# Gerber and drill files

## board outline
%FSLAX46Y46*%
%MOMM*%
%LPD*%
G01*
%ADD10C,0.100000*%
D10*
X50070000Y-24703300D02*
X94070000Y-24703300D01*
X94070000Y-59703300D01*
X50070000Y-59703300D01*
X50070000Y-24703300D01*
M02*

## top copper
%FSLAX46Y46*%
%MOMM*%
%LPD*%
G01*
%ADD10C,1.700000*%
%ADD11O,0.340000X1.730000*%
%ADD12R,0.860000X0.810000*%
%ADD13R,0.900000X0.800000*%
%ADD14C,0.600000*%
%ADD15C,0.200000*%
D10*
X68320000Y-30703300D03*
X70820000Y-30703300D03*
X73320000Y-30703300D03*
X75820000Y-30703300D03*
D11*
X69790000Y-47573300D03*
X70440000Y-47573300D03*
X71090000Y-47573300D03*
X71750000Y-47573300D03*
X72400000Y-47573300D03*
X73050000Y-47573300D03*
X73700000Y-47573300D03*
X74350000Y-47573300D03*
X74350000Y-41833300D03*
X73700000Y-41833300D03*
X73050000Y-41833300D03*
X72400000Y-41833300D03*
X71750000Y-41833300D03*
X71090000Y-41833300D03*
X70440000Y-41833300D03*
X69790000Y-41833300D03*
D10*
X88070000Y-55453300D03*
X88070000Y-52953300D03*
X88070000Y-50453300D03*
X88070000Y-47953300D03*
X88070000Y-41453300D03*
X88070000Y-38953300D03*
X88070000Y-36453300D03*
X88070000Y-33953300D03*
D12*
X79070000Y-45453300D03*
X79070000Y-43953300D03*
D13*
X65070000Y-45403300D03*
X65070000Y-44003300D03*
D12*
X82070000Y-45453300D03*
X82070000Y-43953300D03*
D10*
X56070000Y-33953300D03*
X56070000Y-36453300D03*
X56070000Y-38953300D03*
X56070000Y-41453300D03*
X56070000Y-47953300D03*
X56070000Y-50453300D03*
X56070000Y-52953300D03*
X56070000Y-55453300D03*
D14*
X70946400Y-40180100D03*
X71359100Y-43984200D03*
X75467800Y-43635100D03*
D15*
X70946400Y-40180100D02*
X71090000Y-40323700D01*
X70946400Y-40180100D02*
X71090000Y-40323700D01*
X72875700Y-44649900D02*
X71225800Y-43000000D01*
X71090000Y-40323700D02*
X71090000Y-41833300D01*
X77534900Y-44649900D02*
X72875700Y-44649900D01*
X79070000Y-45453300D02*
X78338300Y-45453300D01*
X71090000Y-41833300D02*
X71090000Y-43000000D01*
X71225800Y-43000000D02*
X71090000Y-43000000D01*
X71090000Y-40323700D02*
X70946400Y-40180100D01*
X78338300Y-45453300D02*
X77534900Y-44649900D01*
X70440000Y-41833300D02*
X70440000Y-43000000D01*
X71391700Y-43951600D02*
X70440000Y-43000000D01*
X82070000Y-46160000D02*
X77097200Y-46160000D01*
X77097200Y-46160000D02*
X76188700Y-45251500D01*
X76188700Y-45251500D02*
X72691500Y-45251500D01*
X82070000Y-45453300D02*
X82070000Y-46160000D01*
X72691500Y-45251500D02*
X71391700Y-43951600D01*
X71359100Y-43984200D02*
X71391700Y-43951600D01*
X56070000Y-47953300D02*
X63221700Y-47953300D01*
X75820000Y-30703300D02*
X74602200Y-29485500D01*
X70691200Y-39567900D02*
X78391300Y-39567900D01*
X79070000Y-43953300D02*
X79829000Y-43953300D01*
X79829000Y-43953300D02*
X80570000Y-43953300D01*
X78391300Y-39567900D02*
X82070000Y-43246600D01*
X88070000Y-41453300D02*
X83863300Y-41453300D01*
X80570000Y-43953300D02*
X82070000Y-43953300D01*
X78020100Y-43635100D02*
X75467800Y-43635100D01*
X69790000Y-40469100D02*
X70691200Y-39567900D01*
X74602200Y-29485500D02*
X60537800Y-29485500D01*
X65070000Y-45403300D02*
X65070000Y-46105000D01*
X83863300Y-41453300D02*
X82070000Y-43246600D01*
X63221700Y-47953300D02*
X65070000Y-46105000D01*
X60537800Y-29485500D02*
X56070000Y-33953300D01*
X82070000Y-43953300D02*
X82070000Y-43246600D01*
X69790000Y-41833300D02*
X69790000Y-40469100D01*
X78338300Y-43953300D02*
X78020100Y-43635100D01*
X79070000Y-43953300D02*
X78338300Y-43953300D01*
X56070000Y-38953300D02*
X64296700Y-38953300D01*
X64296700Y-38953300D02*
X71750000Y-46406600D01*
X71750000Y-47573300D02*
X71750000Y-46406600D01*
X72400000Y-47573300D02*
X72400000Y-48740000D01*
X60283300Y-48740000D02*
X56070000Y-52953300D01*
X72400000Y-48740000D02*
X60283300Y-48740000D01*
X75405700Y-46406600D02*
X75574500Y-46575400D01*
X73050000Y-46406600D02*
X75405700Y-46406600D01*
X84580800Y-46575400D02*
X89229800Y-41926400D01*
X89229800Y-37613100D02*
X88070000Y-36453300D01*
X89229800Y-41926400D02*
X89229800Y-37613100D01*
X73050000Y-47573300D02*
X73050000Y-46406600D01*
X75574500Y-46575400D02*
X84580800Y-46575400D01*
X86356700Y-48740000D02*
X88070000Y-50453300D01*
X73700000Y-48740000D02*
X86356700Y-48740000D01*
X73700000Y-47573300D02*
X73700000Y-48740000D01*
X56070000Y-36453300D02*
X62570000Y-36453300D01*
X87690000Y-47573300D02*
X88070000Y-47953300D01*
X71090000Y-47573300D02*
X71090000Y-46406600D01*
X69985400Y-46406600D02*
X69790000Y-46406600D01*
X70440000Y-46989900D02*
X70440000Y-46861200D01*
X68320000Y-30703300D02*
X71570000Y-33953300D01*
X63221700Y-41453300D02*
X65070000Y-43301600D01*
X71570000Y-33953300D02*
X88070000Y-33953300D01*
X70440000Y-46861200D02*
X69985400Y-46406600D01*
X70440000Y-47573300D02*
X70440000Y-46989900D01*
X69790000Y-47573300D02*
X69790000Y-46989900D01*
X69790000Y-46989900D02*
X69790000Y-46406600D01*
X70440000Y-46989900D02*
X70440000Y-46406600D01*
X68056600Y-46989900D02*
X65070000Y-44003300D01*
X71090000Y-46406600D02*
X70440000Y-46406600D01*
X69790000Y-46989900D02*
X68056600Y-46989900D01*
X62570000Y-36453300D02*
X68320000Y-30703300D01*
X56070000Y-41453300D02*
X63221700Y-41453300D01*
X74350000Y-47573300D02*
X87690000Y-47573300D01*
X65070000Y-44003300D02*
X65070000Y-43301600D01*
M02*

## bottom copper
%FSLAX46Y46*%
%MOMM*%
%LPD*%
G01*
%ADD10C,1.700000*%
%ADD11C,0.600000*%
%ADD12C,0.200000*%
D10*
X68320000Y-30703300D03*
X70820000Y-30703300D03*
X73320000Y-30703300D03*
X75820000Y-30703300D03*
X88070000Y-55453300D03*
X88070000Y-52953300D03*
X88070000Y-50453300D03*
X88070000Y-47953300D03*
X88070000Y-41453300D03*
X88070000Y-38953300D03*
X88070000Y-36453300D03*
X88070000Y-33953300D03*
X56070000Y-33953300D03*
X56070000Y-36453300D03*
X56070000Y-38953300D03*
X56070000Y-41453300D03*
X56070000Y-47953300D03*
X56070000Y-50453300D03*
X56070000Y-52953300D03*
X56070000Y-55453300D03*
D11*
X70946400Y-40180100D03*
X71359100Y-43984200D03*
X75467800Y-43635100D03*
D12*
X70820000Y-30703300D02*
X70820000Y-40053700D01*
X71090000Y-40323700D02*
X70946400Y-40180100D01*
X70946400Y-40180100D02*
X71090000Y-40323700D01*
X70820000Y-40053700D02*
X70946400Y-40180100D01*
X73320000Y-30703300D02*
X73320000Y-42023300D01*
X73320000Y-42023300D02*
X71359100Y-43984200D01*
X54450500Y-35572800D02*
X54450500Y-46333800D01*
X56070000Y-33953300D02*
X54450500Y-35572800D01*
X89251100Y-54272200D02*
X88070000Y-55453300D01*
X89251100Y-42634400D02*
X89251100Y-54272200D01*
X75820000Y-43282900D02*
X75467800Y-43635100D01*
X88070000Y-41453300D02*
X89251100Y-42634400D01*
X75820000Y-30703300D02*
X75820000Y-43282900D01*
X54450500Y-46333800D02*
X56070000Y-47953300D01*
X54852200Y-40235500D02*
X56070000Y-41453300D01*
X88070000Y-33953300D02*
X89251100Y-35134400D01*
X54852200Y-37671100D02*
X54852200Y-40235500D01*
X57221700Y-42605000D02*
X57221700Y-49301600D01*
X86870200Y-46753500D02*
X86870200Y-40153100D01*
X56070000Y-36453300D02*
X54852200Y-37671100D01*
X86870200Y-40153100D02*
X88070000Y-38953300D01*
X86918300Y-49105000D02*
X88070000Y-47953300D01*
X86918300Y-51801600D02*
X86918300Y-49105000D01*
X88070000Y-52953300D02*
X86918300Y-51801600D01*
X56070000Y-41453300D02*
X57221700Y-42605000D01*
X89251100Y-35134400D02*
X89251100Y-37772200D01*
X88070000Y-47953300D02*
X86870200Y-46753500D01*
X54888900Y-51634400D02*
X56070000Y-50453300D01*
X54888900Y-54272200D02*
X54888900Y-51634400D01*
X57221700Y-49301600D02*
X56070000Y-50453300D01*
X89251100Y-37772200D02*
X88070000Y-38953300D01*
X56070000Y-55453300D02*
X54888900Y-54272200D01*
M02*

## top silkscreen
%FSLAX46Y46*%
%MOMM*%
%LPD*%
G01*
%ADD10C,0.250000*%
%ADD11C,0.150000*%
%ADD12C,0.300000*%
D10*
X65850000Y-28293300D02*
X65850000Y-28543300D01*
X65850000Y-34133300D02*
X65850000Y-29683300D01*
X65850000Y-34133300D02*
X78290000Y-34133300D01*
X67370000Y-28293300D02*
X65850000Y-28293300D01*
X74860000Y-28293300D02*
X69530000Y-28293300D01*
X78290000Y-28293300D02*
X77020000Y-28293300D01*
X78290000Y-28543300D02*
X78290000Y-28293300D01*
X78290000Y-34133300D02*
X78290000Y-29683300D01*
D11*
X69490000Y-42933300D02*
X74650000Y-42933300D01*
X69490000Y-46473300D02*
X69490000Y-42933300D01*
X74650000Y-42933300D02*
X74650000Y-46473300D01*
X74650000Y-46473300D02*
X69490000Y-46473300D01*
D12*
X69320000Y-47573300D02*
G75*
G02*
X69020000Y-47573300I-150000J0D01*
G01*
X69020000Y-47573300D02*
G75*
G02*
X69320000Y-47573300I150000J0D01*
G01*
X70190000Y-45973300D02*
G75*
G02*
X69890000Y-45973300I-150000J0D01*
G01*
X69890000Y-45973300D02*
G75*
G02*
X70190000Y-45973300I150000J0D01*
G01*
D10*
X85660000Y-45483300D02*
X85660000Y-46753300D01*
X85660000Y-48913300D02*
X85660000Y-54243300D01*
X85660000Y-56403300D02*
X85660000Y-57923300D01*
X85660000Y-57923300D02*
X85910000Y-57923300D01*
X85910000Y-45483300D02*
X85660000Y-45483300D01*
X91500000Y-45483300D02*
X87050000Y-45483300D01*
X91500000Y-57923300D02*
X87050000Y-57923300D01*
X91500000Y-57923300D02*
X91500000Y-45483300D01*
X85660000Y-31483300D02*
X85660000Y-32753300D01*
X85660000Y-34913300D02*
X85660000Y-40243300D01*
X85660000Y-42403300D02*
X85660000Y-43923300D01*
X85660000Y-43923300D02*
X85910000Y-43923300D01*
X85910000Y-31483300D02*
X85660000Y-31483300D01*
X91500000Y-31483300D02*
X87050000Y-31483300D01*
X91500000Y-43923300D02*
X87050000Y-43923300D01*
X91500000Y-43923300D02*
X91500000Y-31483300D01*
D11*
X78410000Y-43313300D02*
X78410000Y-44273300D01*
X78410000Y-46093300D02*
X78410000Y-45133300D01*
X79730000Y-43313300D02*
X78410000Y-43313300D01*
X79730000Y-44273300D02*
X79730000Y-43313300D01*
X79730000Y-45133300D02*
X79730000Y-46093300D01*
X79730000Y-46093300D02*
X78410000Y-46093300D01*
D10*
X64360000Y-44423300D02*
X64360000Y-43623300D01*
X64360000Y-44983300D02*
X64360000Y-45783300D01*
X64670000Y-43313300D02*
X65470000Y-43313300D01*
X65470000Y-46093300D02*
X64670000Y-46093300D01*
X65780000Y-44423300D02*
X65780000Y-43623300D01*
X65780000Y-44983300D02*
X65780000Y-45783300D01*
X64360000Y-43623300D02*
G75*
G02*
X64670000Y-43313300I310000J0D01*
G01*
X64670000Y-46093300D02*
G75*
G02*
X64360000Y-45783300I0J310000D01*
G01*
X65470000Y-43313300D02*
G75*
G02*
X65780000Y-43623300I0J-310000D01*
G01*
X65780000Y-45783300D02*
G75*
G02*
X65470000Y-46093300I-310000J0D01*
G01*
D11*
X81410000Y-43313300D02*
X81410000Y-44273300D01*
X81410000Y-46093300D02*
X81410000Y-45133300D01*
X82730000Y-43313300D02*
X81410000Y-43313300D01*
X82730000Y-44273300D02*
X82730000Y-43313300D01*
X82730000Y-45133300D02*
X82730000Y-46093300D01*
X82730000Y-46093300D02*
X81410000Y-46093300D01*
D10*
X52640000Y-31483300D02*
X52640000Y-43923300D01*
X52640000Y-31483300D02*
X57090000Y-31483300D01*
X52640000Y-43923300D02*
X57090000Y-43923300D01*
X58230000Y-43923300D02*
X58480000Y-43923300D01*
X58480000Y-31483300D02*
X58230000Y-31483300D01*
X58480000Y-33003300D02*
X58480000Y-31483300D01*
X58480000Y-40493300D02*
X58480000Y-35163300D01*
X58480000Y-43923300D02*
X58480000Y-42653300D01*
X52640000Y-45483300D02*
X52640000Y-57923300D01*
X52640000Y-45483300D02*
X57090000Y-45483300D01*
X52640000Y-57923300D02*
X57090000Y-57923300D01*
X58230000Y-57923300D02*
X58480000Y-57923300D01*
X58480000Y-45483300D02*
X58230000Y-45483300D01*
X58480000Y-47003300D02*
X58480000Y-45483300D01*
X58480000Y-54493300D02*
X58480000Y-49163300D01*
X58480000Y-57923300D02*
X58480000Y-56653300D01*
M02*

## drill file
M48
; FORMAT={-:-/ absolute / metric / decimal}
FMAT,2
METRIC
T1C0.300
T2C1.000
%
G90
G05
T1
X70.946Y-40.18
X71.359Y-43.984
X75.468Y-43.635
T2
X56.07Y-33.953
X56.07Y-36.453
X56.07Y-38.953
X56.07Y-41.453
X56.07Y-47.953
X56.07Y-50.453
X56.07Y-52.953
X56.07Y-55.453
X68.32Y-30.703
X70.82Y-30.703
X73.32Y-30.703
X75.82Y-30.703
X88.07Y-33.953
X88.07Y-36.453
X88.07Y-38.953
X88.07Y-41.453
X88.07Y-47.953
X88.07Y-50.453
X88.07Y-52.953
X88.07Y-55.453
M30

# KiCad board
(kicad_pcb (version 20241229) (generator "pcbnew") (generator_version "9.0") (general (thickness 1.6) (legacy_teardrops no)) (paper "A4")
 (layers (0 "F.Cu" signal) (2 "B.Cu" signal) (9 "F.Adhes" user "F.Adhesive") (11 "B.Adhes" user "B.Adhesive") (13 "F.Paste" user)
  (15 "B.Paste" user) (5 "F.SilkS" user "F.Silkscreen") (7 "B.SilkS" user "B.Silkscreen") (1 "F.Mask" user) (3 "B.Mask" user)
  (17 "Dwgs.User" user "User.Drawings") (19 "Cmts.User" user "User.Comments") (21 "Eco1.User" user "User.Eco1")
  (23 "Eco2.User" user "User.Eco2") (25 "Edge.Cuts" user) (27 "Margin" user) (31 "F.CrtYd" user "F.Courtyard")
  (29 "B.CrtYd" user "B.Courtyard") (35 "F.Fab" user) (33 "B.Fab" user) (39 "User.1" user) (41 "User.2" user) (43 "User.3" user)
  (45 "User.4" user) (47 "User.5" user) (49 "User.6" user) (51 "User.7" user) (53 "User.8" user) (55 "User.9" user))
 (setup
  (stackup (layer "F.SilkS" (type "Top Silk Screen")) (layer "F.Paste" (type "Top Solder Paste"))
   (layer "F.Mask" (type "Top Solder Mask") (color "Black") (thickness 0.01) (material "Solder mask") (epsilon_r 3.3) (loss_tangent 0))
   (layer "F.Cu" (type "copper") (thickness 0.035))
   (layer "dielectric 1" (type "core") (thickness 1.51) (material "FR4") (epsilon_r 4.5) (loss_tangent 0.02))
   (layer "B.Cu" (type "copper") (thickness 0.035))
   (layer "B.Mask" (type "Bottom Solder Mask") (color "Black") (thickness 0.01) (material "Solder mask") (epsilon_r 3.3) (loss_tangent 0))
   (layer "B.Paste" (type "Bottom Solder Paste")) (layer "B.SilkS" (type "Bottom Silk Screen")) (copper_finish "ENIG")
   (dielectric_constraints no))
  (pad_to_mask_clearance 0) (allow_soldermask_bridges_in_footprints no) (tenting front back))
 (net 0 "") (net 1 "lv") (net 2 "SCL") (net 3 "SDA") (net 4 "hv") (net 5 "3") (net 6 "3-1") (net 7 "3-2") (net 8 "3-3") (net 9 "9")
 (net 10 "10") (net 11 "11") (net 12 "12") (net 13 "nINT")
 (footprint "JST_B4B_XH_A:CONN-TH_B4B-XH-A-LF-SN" (layer "F.Cu") (at 72.07 30.7033 180)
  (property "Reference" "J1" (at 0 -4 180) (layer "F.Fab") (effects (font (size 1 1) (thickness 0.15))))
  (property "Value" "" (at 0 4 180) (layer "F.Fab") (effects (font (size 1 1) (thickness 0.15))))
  (fp_line (start 6.22 2.41) (end 6.22 2.16) (stroke (width 0.25) (type solid)) (layer "F.SilkS"))
  (fp_line (start 6.22 -3.43) (end 6.22 1.02) (stroke (width 0.25) (type solid)) (layer "F.SilkS"))
  (fp_line (start 6.22 -3.43) (end -6.22 -3.43) (stroke (width 0.25) (type solid)) (layer "F.SilkS"))
  (fp_line (start 4.7 2.41) (end 6.22 2.41) (stroke (width 0.25) (type solid)) (layer "F.SilkS"))
  (fp_line (start -2.79 2.41) (end 2.54 2.41) (stroke (width 0.25) (type solid)) (layer "F.SilkS"))
  (fp_line (start -6.22 2.41) (end -4.95 2.41) (stroke (width 0.25) (type solid)) (layer "F.SilkS"))
  (fp_line (start -6.22 2.16) (end -6.22 2.41) (stroke (width 0.25) (type solid)) (layer "F.SilkS"))
  (fp_line (start -6.22 -3.43) (end -6.22 1.02) (stroke (width 0.25) (type solid)) (layer "F.SilkS"))
  (pad "1" thru_hole circle (at 3.75 0 180) (size 1.7 1.7) (drill 0.999998) (layers "*.Cu" "*.Mask") (remove_unused_layers no) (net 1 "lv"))
  (pad "2" thru_hole circle (at 1.25 0 180) (size 1.7 1.7) (drill 0.999998) (layers "*.Cu" "*.Mask") (remove_unused_layers no) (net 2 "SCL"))
  (pad "3" thru_hole circle (at -1.25 0 180) (size 1.7 1.7) (drill 0.999998) (layers "*.Cu" "*.Mask") (remove_unused_layers no)
   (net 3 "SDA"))
  (pad "4" thru_hole circle (at -3.75 0 180) (size 1.7 1.7) (drill 0.999998) (layers "*.Cu" "*.Mask") (remove_unused_layers no) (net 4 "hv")))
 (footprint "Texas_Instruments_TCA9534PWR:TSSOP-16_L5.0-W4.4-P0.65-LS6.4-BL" (layer "F.Cu") (at 72.07 44.7033)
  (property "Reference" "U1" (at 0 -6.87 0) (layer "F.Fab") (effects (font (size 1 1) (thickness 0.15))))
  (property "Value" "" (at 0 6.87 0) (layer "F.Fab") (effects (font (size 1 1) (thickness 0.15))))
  (fp_line (start -2.58 -1.77) (end 2.58 -1.77) (stroke (width 0.15) (type solid)) (layer "F.SilkS"))
  (fp_line (start -2.58 1.77) (end -2.58 -1.77) (stroke (width 0.15) (type solid)) (layer "F.SilkS"))
  (fp_line (start 2.58 -1.77) (end 2.58 1.77) (stroke (width 0.15) (type solid)) (layer "F.SilkS"))
  (fp_line (start 2.58 1.77) (end -2.58 1.77) (stroke (width 0.15) (type solid)) (layer "F.SilkS"))
  (fp_circle (center -2.9 2.87) (end -2.75 2.87) (stroke (width 0.3) (type solid)) (fill no) (layer "F.SilkS"))
  (fp_circle (center -2.03 1.27) (end -1.88 1.27) (stroke (width 0.3) (type solid)) (fill no) (layer "F.SilkS"))
  (pad "1" smd oval (at -2.28 2.87) (size 0.34 1.73) (layers "F.Cu" "F.Mask" "F.Paste") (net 1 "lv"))
  (pad "2" smd oval (at -1.63 2.87) (size 0.34 1.73) (layers "F.Cu" "F.Mask" "F.Paste") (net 1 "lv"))
  (pad "3" smd oval (at -0.98 2.87) (size 0.34 1.73) (layers "F.Cu" "F.Mask" "F.Paste") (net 1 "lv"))
  (pad "4" smd oval (at -0.32 2.87) (size 0.34 1.73) (layers "F.Cu" "F.Mask" "F.Paste") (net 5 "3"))
  (pad "5" smd oval (at 0.33 2.87) (size 0.34 1.73) (layers "F.Cu" "F.Mask" "F.Paste") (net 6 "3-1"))
  (pad "6" smd oval (at 0.98 2.87) (size 0.34 1.73) (layers "F.Cu" "F.Mask" "F.Paste") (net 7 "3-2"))
  (pad "7" smd oval (at 1.63 2.87) (size 0.34 1.73) (layers "F.Cu" "F.Mask" "F.Paste") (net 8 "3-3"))
  (pad "8" smd oval (at 2.28 2.87) (size 0.34 1.73) (layers "F.Cu" "F.Mask" "F.Paste") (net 1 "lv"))
  (pad "9" smd oval (at 2.28 -2.87) (size 0.34 1.73) (layers "F.Cu" "F.Mask" "F.Paste") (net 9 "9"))
  (pad "10" smd oval (at 1.63 -2.87) (size 0.34 1.73) (layers "F.Cu" "F.Mask" "F.Paste") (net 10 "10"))
  (pad "11" smd oval (at 0.98 -2.87) (size 0.34 1.73) (layers "F.Cu" "F.Mask" "F.Paste") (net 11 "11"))
  (pad "12" smd oval (at 0.33 -2.87) (size 0.34 1.73) (layers "F.Cu" "F.Mask" "F.Paste") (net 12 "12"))
  (pad "13" smd oval (at -0.32 -2.87) (size 0.34 1.73) (layers "F.Cu" "F.Mask" "F.Paste") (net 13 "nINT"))
  (pad "14" smd oval (at -0.98 -2.87) (size 0.34 1.73) (layers "F.Cu" "F.Mask" "F.Paste") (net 2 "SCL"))
  (pad "15" smd oval (at -1.63 -2.87) (size 0.34 1.73) (layers "F.Cu" "F.Mask" "F.Paste") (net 3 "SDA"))
  (pad "16" smd oval (at -2.28 -2.87) (size 0.34 1.73) (layers "F.Cu" "F.Mask" "F.Paste") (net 4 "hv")))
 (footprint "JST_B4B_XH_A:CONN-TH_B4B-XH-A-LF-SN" (layer "F.Cu") (at 88.07 51.7033 -90)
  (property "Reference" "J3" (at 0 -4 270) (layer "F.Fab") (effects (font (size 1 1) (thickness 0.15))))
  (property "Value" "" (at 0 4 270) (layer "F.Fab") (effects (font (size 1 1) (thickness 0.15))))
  (fp_line (start -6.22 2.41) (end -4.95 2.41) (stroke (width 0.25) (type solid)) (layer "F.SilkS"))
  (fp_line (start -2.79 2.41) (end 2.54 2.41) (stroke (width 0.25) (type solid)) (layer "F.SilkS"))
  (fp_line (start 4.7 2.41) (end 6.22 2.41) (stroke (width 0.25) (type solid)) (layer "F.SilkS"))
  (fp_line (start 6.22 2.41) (end 6.22 2.16) (stroke (width 0.25) (type solid)) (layer "F.SilkS"))
  (fp_line (start -6.22 2.16) (end -6.22 2.41) (stroke (width 0.25) (type solid)) (layer "F.SilkS"))
  (fp_line (start -6.22 -3.43) (end -6.22 1.02) (stroke (width 0.25) (type solid)) (layer "F.SilkS"))
  (fp_line (start 6.22 -3.43) (end 6.22 1.02) (stroke (width 0.25) (type solid)) (layer "F.SilkS"))
  (fp_line (start 6.22 -3.43) (end -6.22 -3.43) (stroke (width 0.25) (type solid)) (layer "F.SilkS"))
  (pad "1" thru_hole circle (at 3.75 0 270) (size 1.7 1.7) (drill 0.999998) (layers "*.Cu" "*.Mask") (remove_unused_layers no) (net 4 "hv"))
  (pad "2" thru_hole circle (at 1.25 0 270) (size 1.7 1.7) (drill 0.999998) (layers "*.Cu" "*.Mask") (remove_unused_layers no) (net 1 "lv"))
  (pad "3" thru_hole circle (at -1.25 0 270) (size 1.7 1.7) (drill 0.999998) (layers "*.Cu" "*.Mask") (remove_unused_layers no)
   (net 8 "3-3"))
  (pad "4" thru_hole circle (at -3.75 0 270) (size 1.7 1.7) (drill 0.999998) (layers "*.Cu" "*.Mask") (remove_unused_layers no) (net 1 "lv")))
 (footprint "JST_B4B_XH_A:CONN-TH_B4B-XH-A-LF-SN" (layer "F.Cu") (at 88.07 37.7033 -90)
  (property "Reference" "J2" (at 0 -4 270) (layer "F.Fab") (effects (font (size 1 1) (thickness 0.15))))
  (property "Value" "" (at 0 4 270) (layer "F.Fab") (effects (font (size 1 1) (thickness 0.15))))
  (fp_line (start -6.22 2.41) (end -4.95 2.41) (stroke (width 0.25) (type solid)) (layer "F.SilkS"))
  (fp_line (start -2.79 2.41) (end 2.54 2.41) (stroke (width 0.25) (type solid)) (layer "F.SilkS"))
  (fp_line (start 4.7 2.41) (end 6.22 2.41) (stroke (width 0.25) (type solid)) (layer "F.SilkS"))
  (fp_line (start 6.22 2.41) (end 6.22 2.16) (stroke (width 0.25) (type solid)) (layer "F.SilkS"))
  (fp_line (start -6.22 2.16) (end -6.22 2.41) (stroke (width 0.25) (type solid)) (layer "F.SilkS"))
  (fp_line (start -6.22 -3.43) (end -6.22 1.02) (stroke (width 0.25) (type solid)) (layer "F.SilkS"))
  (fp_line (start 6.22 -3.43) (end 6.22 1.02) (stroke (width 0.25) (type solid)) (layer "F.SilkS"))
  (fp_line (start 6.22 -3.43) (end -6.22 -3.43) (stroke (width 0.25) (type solid)) (layer "F.SilkS"))
  (pad "1" thru_hole circle (at 3.75 0 270) (size 1.7 1.7) (drill 0.999998) (layers "*.Cu" "*.Mask") (remove_unused_layers no) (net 4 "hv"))
  (pad "2" thru_hole circle (at 1.25 0 270) (size 1.7 1.7) (drill 0.999998) (layers "*.Cu" "*.Mask") (remove_unused_layers no) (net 1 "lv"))
  (pad "3" thru_hole circle (at -1.25 0 270) (size 1.7 1.7) (drill 0.999998) (layers "*.Cu" "*.Mask") (remove_unused_layers no)
   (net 7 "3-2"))
  (pad "4" thru_hole circle (at -3.75 0 270) (size 1.7 1.7) (drill 0.999998) (layers "*.Cu" "*.Mask") (remove_unused_layers no) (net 1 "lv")))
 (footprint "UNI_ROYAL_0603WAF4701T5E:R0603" (layer "F.Cu") (at 79.07 44.7033 90)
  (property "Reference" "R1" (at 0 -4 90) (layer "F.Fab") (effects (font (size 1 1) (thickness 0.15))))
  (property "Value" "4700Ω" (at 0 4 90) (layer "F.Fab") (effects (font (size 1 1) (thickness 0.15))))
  (fp_line (start 1.39 -0.66) (end 0.43 -0.66) (stroke (width 0.15) (type solid)) (layer "F.SilkS"))
  (fp_line (start -1.39 -0.66) (end -0.43 -0.66) (stroke (width 0.15) (type solid)) (layer "F.SilkS"))
  (fp_line (start 1.39 0.66) (end 1.39 -0.66) (stroke (width 0.15) (type solid)) (layer "F.SilkS"))
  (fp_line (start 0.43 0.66) (end 1.39 0.66) (stroke (width 0.15) (type solid)) (layer "F.SilkS"))
  (fp_line (start -0.43 0.66) (end -1.39 0.66) (stroke (width 0.15) (type solid)) (layer "F.SilkS"))
  (fp_line (start -1.39 0.66) (end -1.39 -0.66) (stroke (width 0.15) (type solid)) (layer "F.SilkS"))
  (pad "1" smd rect (at -0.75 0 90) (size 0.81 0.86) (layers "F.Cu" "F.Mask" "F.Paste") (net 2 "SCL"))
  (pad "2" smd rect (at 0.75 0 90) (size 0.81 0.86) (layers "F.Cu" "F.Mask" "F.Paste") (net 4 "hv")))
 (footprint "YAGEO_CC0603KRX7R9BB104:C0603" (layer "F.Cu") (at 65.07 44.7033 90)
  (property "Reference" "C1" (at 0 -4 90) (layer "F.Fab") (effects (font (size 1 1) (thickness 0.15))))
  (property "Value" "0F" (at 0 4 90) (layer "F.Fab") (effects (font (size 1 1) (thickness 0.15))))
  (fp_line (start 0.28 -0.71) (end 1.08 -0.71) (stroke (width 0.25) (type solid)) (layer "F.SilkS"))
  (fp_line (start -0.28 -0.71) (end -1.08 -0.71) (stroke (width 0.25) (type solid)) (layer "F.SilkS"))
  (fp_line (start 1.39 -0.4) (end 1.39 0.4) (stroke (width 0.25) (type solid)) (layer "F.SilkS"))
  (fp_line (start -1.39 0.4) (end -1.39 -0.4) (stroke (width 0.25) (type solid)) (layer "F.SilkS"))
  (fp_line (start 0.28 0.71) (end 1.08 0.71) (stroke (width 0.25) (type solid)) (layer "F.SilkS"))
  (fp_line (start -0.28 0.71) (end -1.08 0.71) (stroke (width 0.25) (type solid)) (layer "F.SilkS"))
  (fp_arc (start 1.08 -0.71) (mid 1.299203 -0.619203) (end 1.39 -0.4) (stroke (width 0.25) (type solid)) (layer "F.SilkS"))
  (fp_arc (start -1.39 -0.4) (mid -1.299203 -0.619203) (end -1.08 -0.71) (stroke (width 0.25) (type solid)) (layer "F.SilkS"))
  (fp_arc (start 1.39 0.4) (mid 1.299203 0.619203) (end 1.08 0.71) (stroke (width 0.25) (type solid)) (layer "F.SilkS"))
  (fp_arc (start -1.08 0.71) (mid -1.299203 0.619203) (end -1.39 0.4) (stroke (width 0.25) (type solid)) (layer "F.SilkS"))
  (pad "1" smd rect (at -0.7 0 90) (size 0.8 0.9) (layers "F.Cu" "F.Mask" "F.Paste") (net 4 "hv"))
  (pad "2" smd rect (at 0.7 0 90) (size 0.8 0.9) (layers "F.Cu" "F.Mask" "F.Paste") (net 1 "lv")))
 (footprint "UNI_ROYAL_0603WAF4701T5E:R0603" (layer "F.Cu") (at 82.07 44.7033 90)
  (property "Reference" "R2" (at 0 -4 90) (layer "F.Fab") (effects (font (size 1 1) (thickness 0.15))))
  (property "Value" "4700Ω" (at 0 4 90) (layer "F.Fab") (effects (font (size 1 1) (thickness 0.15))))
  (fp_line (start 1.39 -0.66) (end 0.43 -0.66) (stroke (width 0.15) (type solid)) (layer "F.SilkS"))
  (fp_line (start -1.39 -0.66) (end -0.43 -0.66) (stroke (width 0.15) (type solid)) (layer "F.SilkS"))
  (fp_line (start 1.39 0.66) (end 1.39 -0.66) (stroke (width 0.15) (type solid)) (layer "F.SilkS"))
  (fp_line (start 0.43 0.66) (end 1.39 0.66) (stroke (width 0.15) (type solid)) (layer "F.SilkS"))
  (fp_line (start -0.43 0.66) (end -1.39 0.66) (stroke (width 0.15) (type solid)) (layer "F.SilkS"))
  (fp_line (start -1.39 0.66) (end -1.39 -0.66) (stroke (width 0.15) (type solid)) (layer "F.SilkS"))
  (pad "1" smd rect (at -0.75 0 90) (size 0.81 0.86) (layers "F.Cu" "F.Mask" "F.Paste") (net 3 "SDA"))
  (pad "2" smd rect (at 0.75 0 90) (size 0.81 0.86) (layers "F.Cu" "F.Mask" "F.Paste") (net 4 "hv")))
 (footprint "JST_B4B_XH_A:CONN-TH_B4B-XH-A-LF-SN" (layer "F.Cu") (at 56.07 37.7033 90)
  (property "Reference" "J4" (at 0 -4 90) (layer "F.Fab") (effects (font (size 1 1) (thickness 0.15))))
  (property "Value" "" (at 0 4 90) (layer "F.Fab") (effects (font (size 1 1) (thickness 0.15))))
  (fp_line (start 6.22 -3.43) (end -6.22 -3.43) (stroke (width 0.25) (type solid)) (layer "F.SilkS"))
  (fp_line (start 6.22 -3.43) (end 6.22 1.02) (stroke (width 0.25) (type solid)) (layer "F.SilkS"))
  (fp_line (start -6.22 -3.43) (end -6.22 1.02) (stroke (width 0.25) (type solid)) (layer "F.SilkS"))
  (fp_line (start -6.22 2.16) (end -6.22 2.41) (stroke (width 0.25) (type solid)) (layer "F.SilkS"))
  (fp_line (start 6.22 2.41) (end 6.22 2.16) (stroke (width 0.25) (type solid)) (layer "F.SilkS"))
  (fp_line (start 4.7 2.41) (end 6.22 2.41) (stroke (width 0.25) (type solid)) (layer "F.SilkS"))
  (fp_line (start -2.79 2.41) (end 2.54 2.41) (stroke (width 0.25) (type solid)) (layer "F.SilkS"))
  (fp_line (start -6.22 2.41) (end -4.95 2.41) (stroke (width 0.25) (type solid)) (layer "F.SilkS"))
  (pad "1" thru_hole circle (at 3.75 0 90) (size 1.7 1.7) (drill 0.999998) (layers "*.Cu" "*.Mask") (remove_unused_layers no) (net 4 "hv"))
  (pad "2" thru_hole circle (at 1.25 0 90) (size 1.7 1.7) (drill 0.999998) (layers "*.Cu" "*.Mask") (remove_unused_layers no) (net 1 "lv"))
  (pad "3" thru_hole circle (at -1.25 0 90) (size 1.7 1.7) (drill 0.999998) (layers "*.Cu" "*.Mask") (remove_unused_layers no) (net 5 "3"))
  (pad "4" thru_hole circle (at -3.75 0 90) (size 1.7 1.7) (drill 0.999998) (layers "*.Cu" "*.Mask") (remove_unused_layers no) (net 1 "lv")))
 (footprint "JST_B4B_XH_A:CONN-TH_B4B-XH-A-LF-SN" (layer "F.Cu") (at 56.07 51.7033 90)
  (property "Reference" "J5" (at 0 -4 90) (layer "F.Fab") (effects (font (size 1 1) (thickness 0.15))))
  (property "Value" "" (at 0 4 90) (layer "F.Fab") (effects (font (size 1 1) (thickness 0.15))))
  (fp_line (start 6.22 -3.43) (end -6.22 -3.43) (stroke (width 0.25) (type solid)) (layer "F.SilkS"))
  (fp_line (start 6.22 -3.43) (end 6.22 1.02) (stroke (width 0.25) (type solid)) (layer "F.SilkS"))
  (fp_line (start -6.22 -3.43) (end -6.22 1.02) (stroke (width 0.25) (type solid)) (layer "F.SilkS"))
  (fp_line (start -6.22 2.16) (end -6.22 2.41) (stroke (width 0.25) (type solid)) (layer "F.SilkS"))
  (fp_line (start 6.22 2.41) (end 6.22 2.16) (stroke (width 0.25) (type solid)) (layer "F.SilkS"))
  (fp_line (start 4.7 2.41) (end 6.22 2.41) (stroke (width 0.25) (type solid)) (layer "F.SilkS"))
  (fp_line (start -2.79 2.41) (end 2.54 2.41) (stroke (width 0.25) (type solid)) (layer "F.SilkS"))
  (fp_line (start -6.22 2.41) (end -4.95 2.41) (stroke (width 0.25) (type solid)) (layer "F.SilkS"))
  (pad "1" thru_hole circle (at 3.75 0 90) (size 1.7 1.7) (drill 0.999998) (layers "*.Cu" "*.Mask") (remove_unused_layers no) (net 4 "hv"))
  (pad "2" thru_hole circle (at 1.25 0 90) (size 1.7 1.7) (drill 0.999998) (layers "*.Cu" "*.Mask") (remove_unused_layers no) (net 1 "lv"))
  (pad "3" thru_hole circle (at -1.25 0 90) (size 1.7 1.7) (drill 0.999998) (layers "*.Cu" "*.Mask") (remove_unused_layers no) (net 6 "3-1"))
  (pad "4" thru_hole circle (at -3.75 0 90) (size 1.7 1.7) (drill 0.999998) (layers "*.Cu" "*.Mask") (remove_unused_layers no) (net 1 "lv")))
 (gr_rect (start 50.07 24.7033) (end 94.07 59.7033) (stroke (width 0.1) (type solid)) (fill no) (layer "Edge.Cuts"))
 (segment (start 70.9464 40.1801) (end 71.09 40.3237) (width 0.2) (layer "F.Cu") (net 2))
 (segment (start 70.9464 40.1801) (end 71.09 40.3237) (width 0.2) (layer "F.Cu") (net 2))
 (segment (start 72.8757 44.6499) (end 71.2258 43) (width 0.2) (layer "F.Cu") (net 2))
 (segment (start 71.09 40.3237) (end 71.09 41.8333) (width 0.2) (layer "F.Cu") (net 2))
 (segment (start 77.5349 44.6499) (end 72.8757 44.6499) (width 0.2) (layer "F.Cu") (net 2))
 (segment (start 79.07 45.4533) (end 78.3383 45.4533) (width 0.2) (layer "F.Cu") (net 2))
 (segment (start 71.09 41.8333) (end 71.09 43) (width 0.2) (layer "F.Cu") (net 2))
 (segment (start 71.2258 43) (end 71.09 43) (width 0.2) (layer "F.Cu") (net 2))
 (segment (start 71.09 40.3237) (end 70.9464 40.1801) (width 0.2) (layer "F.Cu") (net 2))
 (segment (start 78.3383 45.4533) (end 77.5349 44.6499) (width 0.2) (layer "F.Cu") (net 2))
 (via (at 70.9464 40.1801) (size 0.6) (drill 0.3) (layers "F.Cu" "B.Cu") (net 2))
 (segment (start 70.82 30.7033) (end 70.82 40.0537) (width 0.2) (layer "B.Cu") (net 2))
 (segment (start 71.09 40.3237) (end 70.9464 40.1801) (width 0.2) (layer "B.Cu") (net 2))
 (segment (start 70.9464 40.1801) (end 71.09 40.3237) (width 0.2) (layer "B.Cu") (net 2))
 (segment (start 70.82 40.0537) (end 70.9464 40.1801) (width 0.2) (layer "B.Cu") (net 2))
 (segment (start 70.44 41.8333) (end 70.44 43) (width 0.2) (layer "F.Cu") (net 3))
 (segment (start 71.3917 43.9516) (end 70.44 43) (width 0.2) (layer "F.Cu") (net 3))
 (segment (start 82.07 46.16) (end 77.0972 46.16) (width 0.2) (layer "F.Cu") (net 3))
 (segment (start 77.0972 46.16) (end 76.1887 45.2515) (width 0.2) (layer "F.Cu") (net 3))
 (segment (start 76.1887 45.2515) (end 72.6915 45.2515) (width 0.2) (layer "F.Cu") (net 3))
 (segment (start 82.07 45.4533) (end 82.07 46.16) (width 0.2) (layer "F.Cu") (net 3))
 (segment (start 72.6915 45.2515) (end 71.3917 43.9516) (width 0.2) (layer "F.Cu") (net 3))
 (segment (start 71.3591 43.9842) (end 71.3917 43.9516) (width 0.2) (layer "F.Cu") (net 3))
 (via (at 71.3591 43.9842) (size 0.6) (drill 0.3) (layers "F.Cu" "B.Cu") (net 3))
 (segment (start 73.32 30.7033) (end 73.32 42.0233) (width 0.2) (layer "B.Cu") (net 3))
 (segment (start 73.32 42.0233) (end 71.3591 43.9842) (width 0.2) (layer "B.Cu") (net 3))
 (segment (start 56.07 47.9533) (end 63.2217 47.9533) (width 0.2) (layer "F.Cu") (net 4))
 (segment (start 75.82 30.7033) (end 74.6022 29.4855) (width 0.2) (layer "F.Cu") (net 4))
 (segment (start 70.6912 39.5679) (end 78.3913 39.5679) (width 0.2) (layer "F.Cu") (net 4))
 (segment (start 79.07 43.9533) (end 79.829 43.9533) (width 0.2) (layer "F.Cu") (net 4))
 (segment (start 79.829 43.9533) (end 80.57 43.9533) (width 0.2) (layer "F.Cu") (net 4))
 (segment (start 78.3913 39.5679) (end 82.07 43.2466) (width 0.2) (layer "F.Cu") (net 4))
 (segment (start 88.07 41.4533) (end 83.8633 41.4533) (width 0.2) (layer "F.Cu") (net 4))
 (segment (start 80.57 43.9533) (end 82.07 43.9533) (width 0.2) (layer "F.Cu") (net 4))
 (segment (start 78.0201 43.6351) (end 75.4678 43.6351) (width 0.2) (layer "F.Cu") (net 4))
 (segment (start 69.79 40.4691) (end 70.6912 39.5679) (width 0.2) (layer "F.Cu") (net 4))
 (segment (start 74.6022 29.4855) (end 60.5378 29.4855) (width 0.2) (layer "F.Cu") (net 4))
 (segment (start 65.07 45.4033) (end 65.07 46.105) (width 0.2) (layer "F.Cu") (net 4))
 (segment (start 83.8633 41.4533) (end 82.07 43.2466) (width 0.2) (layer "F.Cu") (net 4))
 (segment (start 63.2217 47.9533) (end 65.07 46.105) (width 0.2) (layer "F.Cu") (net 4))
 (segment (start 60.5378 29.4855) (end 56.07 33.9533) (width 0.2) (layer "F.Cu") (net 4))
 (segment (start 82.07 43.9533) (end 82.07 43.2466) (width 0.2) (layer "F.Cu") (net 4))
 (segment (start 69.79 41.8333) (end 69.79 40.4691) (width 0.2) (layer "F.Cu") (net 4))
 (segment (start 78.3383 43.9533) (end 78.0201 43.6351) (width 0.2) (layer "F.Cu") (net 4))
 (segment (start 79.07 43.9533) (end 78.3383 43.9533) (width 0.2) (layer "F.Cu") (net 4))
 (via (at 75.4678 43.6351) (size 0.6) (drill 0.3) (layers "F.Cu" "B.Cu") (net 4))
 (segment (start 54.4505 35.5728) (end 54.4505 46.3338) (width 0.2) (layer "B.Cu") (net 4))
 (segment (start 56.07 33.9533) (end 54.4505 35.5728) (width 0.2) (layer "B.Cu") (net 4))
 (segment (start 89.2511 54.2722) (end 88.07 55.4533) (width 0.2) (layer "B.Cu") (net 4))
 (segment (start 89.2511 42.6344) (end 89.2511 54.2722) (width 0.2) (layer "B.Cu") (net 4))
 (segment (start 75.82 43.2829) (end 75.4678 43.6351) (width 0.2) (layer "B.Cu") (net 4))
 (segment (start 88.07 41.4533) (end 89.2511 42.6344) (width 0.2) (layer "B.Cu") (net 4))
 (segment (start 75.82 30.7033) (end 75.82 43.2829) (width 0.2) (layer "B.Cu") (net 4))
 (segment (start 54.4505 46.3338) (end 56.07 47.9533) (width 0.2) (layer "B.Cu") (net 4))
 (segment (start 56.07 38.9533) (end 64.2967 38.9533) (width 0.2) (layer "F.Cu") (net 5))
 (segment (start 64.2967 38.9533) (end 71.75 46.4066) (width 0.2) (layer "F.Cu") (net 5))
 (segment (start 71.75 47.5733) (end 71.75 46.4066) (width 0.2) (layer "F.Cu") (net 5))
 (segment (start 72.4 47.5733) (end 72.4 48.74) (width 0.2) (layer "F.Cu") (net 6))
 (segment (start 60.2833 48.74) (end 56.07 52.9533) (width 0.2) (layer "F.Cu") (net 6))
 (segment (start 72.4 48.74) (end 60.2833 48.74) (width 0.2) (layer "F.Cu") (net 6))
 (segment (start 75.4057 46.4066) (end 75.5745 46.5754) (width 0.2) (layer "F.Cu") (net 7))
 (segment (start 73.05 46.4066) (end 75.4057 46.4066) (width 0.2) (layer "F.Cu") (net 7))
 (segment (start 84.5808 46.5754) (end 89.2298 41.9264) (width 0.2) (layer "F.Cu") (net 7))
 (segment (start 89.2298 37.6131) (end 88.07 36.4533) (width 0.2) (layer "F.Cu") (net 7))
 (segment (start 89.2298 41.9264) (end 89.2298 37.6131) (width 0.2) (layer "F.Cu") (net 7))
 (segment (start 73.05 47.5733) (end 73.05 46.4066) (width 0.2) (layer "F.Cu") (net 7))
 (segment (start 75.5745 46.5754) (end 84.5808 46.5754) (width 0.2) (layer "F.Cu") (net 7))
 (segment (start 86.3567 48.74) (end 88.07 50.4533) (width 0.2) (layer "F.Cu") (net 8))
 (segment (start 73.7 48.74) (end 86.3567 48.74) (width 0.2) (layer "F.Cu") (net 8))
 (segment (start 73.7 47.5733) (end 73.7 48.74) (width 0.2) (layer "F.Cu") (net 8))
 (segment (start 56.07 36.4533) (end 62.57 36.4533) (width 0.2) (layer "F.Cu") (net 1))
 (segment (start 87.69 47.5733) (end 88.07 47.9533) (width 0.2) (layer "F.Cu") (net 1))
 (segment (start 71.09 47.5733) (end 71.09 46.4066) (width 0.2) (layer "F.Cu") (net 1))
 (segment (start 69.9854 46.4066) (end 69.79 46.4066) (width 0.2) (layer "F.Cu") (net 1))
 (segment (start 70.44 46.9899) (end 70.44 46.8612) (width 0.2) (layer "F.Cu") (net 1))
 (segment (start 68.32 30.7033) (end 71.57 33.9533) (width 0.2) (layer "F.Cu") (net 1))
 (segment (start 63.2217 41.4533) (end 65.07 43.3016) (width 0.2) (layer "F.Cu") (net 1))
 (segment (start 71.57 33.9533) (end 88.07 33.9533) (width 0.2) (layer "F.Cu") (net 1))
 (segment (start 70.44 46.8612) (end 69.9854 46.4066) (width 0.2) (layer "F.Cu") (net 1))
 (segment (start 70.44 47.5733) (end 70.44 46.9899) (width 0.2) (layer "F.Cu") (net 1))
 (segment (start 69.79 47.5733) (end 69.79 46.9899) (width 0.2) (layer "F.Cu") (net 1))
 (segment (start 69.79 46.9899) (end 69.79 46.4066) (width 0.2) (layer "F.Cu") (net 1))
 (segment (start 70.44 46.9899) (end 70.44 46.4066) (width 0.2) (layer "F.Cu") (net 1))
 (segment (start 68.0566 46.9899) (end 65.07 44.0033) (width 0.2) (layer "F.Cu") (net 1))
 (segment (start 71.09 46.4066) (end 70.44 46.4066) (width 0.2) (layer "F.Cu") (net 1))
 (segment (start 69.79 46.9899) (end 68.0566 46.9899) (width 0.2) (layer "F.Cu") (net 1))
 (segment (start 62.57 36.4533) (end 68.32 30.7033) (width 0.2) (layer "F.Cu") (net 1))
 (segment (start 56.07 41.4533) (end 63.2217 41.4533) (width 0.2) (layer "F.Cu") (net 1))
 (segment (start 74.35 47.5733) (end 87.69 47.5733) (width 0.2) (layer "F.Cu") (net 1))
 (segment (start 65.07 44.0033) (end 65.07 43.3016) (width 0.2) (layer "F.Cu") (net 1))
 (segment (start 54.8522 40.2355) (end 56.07 41.4533) (width 0.2) (layer "B.Cu") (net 1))
 (segment (start 88.07 33.9533) (end 89.2511 35.1344) (width 0.2) (layer "B.Cu") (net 1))
 (segment (start 54.8522 37.6711) (end 54.8522 40.2355) (width 0.2) (layer "B.Cu") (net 1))
 (segment (start 57.2217 42.605) (end 57.2217 49.3016) (width 0.2) (layer "B.Cu") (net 1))
 (segment (start 86.8702 46.7535) (end 86.8702 40.1531) (width 0.2) (layer "B.Cu") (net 1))
 (segment (start 56.07 36.4533) (end 54.8522 37.6711) (width 0.2) (layer "B.Cu") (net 1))
 (segment (start 86.8702 40.1531) (end 88.07 38.9533) (width 0.2) (layer "B.Cu") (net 1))
 (segment (start 86.9183 49.105) (end 88.07 47.9533) (width 0.2) (layer "B.Cu") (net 1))
 (segment (start 86.9183 51.8016) (end 86.9183 49.105) (width 0.2) (layer "B.Cu") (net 1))
 (segment (start 88.07 52.9533) (end 86.9183 51.8016) (width 0.2) (layer "B.Cu") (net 1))
 (segment (start 56.07 41.4533) (end 57.2217 42.605) (width 0.2) (layer "B.Cu") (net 1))
 (segment (start 89.2511 35.1344) (end 89.2511 37.7722) (width 0.2) (layer "B.Cu") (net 1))
 (segment (start 88.07 47.9533) (end 86.8702 46.7535) (width 0.2) (layer "B.Cu") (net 1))
 (segment (start 54.8889 51.6344) (end 56.07 50.4533) (width 0.2) (layer "B.Cu") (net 1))
 (segment (start 54.8889 54.2722) (end 54.8889 51.6344) (width 0.2) (layer "B.Cu") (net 1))
 (segment (start 57.2217 49.3016) (end 56.07 50.4533) (width 0.2) (layer "B.Cu") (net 1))
 (segment (start 89.2511 37.7722) (end 88.07 38.9533) (width 0.2) (layer "B.Cu") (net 1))
 (segment (start 56.07 55.4533) (end 54.8889 54.2722) (width 0.2) (layer "B.Cu") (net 1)))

